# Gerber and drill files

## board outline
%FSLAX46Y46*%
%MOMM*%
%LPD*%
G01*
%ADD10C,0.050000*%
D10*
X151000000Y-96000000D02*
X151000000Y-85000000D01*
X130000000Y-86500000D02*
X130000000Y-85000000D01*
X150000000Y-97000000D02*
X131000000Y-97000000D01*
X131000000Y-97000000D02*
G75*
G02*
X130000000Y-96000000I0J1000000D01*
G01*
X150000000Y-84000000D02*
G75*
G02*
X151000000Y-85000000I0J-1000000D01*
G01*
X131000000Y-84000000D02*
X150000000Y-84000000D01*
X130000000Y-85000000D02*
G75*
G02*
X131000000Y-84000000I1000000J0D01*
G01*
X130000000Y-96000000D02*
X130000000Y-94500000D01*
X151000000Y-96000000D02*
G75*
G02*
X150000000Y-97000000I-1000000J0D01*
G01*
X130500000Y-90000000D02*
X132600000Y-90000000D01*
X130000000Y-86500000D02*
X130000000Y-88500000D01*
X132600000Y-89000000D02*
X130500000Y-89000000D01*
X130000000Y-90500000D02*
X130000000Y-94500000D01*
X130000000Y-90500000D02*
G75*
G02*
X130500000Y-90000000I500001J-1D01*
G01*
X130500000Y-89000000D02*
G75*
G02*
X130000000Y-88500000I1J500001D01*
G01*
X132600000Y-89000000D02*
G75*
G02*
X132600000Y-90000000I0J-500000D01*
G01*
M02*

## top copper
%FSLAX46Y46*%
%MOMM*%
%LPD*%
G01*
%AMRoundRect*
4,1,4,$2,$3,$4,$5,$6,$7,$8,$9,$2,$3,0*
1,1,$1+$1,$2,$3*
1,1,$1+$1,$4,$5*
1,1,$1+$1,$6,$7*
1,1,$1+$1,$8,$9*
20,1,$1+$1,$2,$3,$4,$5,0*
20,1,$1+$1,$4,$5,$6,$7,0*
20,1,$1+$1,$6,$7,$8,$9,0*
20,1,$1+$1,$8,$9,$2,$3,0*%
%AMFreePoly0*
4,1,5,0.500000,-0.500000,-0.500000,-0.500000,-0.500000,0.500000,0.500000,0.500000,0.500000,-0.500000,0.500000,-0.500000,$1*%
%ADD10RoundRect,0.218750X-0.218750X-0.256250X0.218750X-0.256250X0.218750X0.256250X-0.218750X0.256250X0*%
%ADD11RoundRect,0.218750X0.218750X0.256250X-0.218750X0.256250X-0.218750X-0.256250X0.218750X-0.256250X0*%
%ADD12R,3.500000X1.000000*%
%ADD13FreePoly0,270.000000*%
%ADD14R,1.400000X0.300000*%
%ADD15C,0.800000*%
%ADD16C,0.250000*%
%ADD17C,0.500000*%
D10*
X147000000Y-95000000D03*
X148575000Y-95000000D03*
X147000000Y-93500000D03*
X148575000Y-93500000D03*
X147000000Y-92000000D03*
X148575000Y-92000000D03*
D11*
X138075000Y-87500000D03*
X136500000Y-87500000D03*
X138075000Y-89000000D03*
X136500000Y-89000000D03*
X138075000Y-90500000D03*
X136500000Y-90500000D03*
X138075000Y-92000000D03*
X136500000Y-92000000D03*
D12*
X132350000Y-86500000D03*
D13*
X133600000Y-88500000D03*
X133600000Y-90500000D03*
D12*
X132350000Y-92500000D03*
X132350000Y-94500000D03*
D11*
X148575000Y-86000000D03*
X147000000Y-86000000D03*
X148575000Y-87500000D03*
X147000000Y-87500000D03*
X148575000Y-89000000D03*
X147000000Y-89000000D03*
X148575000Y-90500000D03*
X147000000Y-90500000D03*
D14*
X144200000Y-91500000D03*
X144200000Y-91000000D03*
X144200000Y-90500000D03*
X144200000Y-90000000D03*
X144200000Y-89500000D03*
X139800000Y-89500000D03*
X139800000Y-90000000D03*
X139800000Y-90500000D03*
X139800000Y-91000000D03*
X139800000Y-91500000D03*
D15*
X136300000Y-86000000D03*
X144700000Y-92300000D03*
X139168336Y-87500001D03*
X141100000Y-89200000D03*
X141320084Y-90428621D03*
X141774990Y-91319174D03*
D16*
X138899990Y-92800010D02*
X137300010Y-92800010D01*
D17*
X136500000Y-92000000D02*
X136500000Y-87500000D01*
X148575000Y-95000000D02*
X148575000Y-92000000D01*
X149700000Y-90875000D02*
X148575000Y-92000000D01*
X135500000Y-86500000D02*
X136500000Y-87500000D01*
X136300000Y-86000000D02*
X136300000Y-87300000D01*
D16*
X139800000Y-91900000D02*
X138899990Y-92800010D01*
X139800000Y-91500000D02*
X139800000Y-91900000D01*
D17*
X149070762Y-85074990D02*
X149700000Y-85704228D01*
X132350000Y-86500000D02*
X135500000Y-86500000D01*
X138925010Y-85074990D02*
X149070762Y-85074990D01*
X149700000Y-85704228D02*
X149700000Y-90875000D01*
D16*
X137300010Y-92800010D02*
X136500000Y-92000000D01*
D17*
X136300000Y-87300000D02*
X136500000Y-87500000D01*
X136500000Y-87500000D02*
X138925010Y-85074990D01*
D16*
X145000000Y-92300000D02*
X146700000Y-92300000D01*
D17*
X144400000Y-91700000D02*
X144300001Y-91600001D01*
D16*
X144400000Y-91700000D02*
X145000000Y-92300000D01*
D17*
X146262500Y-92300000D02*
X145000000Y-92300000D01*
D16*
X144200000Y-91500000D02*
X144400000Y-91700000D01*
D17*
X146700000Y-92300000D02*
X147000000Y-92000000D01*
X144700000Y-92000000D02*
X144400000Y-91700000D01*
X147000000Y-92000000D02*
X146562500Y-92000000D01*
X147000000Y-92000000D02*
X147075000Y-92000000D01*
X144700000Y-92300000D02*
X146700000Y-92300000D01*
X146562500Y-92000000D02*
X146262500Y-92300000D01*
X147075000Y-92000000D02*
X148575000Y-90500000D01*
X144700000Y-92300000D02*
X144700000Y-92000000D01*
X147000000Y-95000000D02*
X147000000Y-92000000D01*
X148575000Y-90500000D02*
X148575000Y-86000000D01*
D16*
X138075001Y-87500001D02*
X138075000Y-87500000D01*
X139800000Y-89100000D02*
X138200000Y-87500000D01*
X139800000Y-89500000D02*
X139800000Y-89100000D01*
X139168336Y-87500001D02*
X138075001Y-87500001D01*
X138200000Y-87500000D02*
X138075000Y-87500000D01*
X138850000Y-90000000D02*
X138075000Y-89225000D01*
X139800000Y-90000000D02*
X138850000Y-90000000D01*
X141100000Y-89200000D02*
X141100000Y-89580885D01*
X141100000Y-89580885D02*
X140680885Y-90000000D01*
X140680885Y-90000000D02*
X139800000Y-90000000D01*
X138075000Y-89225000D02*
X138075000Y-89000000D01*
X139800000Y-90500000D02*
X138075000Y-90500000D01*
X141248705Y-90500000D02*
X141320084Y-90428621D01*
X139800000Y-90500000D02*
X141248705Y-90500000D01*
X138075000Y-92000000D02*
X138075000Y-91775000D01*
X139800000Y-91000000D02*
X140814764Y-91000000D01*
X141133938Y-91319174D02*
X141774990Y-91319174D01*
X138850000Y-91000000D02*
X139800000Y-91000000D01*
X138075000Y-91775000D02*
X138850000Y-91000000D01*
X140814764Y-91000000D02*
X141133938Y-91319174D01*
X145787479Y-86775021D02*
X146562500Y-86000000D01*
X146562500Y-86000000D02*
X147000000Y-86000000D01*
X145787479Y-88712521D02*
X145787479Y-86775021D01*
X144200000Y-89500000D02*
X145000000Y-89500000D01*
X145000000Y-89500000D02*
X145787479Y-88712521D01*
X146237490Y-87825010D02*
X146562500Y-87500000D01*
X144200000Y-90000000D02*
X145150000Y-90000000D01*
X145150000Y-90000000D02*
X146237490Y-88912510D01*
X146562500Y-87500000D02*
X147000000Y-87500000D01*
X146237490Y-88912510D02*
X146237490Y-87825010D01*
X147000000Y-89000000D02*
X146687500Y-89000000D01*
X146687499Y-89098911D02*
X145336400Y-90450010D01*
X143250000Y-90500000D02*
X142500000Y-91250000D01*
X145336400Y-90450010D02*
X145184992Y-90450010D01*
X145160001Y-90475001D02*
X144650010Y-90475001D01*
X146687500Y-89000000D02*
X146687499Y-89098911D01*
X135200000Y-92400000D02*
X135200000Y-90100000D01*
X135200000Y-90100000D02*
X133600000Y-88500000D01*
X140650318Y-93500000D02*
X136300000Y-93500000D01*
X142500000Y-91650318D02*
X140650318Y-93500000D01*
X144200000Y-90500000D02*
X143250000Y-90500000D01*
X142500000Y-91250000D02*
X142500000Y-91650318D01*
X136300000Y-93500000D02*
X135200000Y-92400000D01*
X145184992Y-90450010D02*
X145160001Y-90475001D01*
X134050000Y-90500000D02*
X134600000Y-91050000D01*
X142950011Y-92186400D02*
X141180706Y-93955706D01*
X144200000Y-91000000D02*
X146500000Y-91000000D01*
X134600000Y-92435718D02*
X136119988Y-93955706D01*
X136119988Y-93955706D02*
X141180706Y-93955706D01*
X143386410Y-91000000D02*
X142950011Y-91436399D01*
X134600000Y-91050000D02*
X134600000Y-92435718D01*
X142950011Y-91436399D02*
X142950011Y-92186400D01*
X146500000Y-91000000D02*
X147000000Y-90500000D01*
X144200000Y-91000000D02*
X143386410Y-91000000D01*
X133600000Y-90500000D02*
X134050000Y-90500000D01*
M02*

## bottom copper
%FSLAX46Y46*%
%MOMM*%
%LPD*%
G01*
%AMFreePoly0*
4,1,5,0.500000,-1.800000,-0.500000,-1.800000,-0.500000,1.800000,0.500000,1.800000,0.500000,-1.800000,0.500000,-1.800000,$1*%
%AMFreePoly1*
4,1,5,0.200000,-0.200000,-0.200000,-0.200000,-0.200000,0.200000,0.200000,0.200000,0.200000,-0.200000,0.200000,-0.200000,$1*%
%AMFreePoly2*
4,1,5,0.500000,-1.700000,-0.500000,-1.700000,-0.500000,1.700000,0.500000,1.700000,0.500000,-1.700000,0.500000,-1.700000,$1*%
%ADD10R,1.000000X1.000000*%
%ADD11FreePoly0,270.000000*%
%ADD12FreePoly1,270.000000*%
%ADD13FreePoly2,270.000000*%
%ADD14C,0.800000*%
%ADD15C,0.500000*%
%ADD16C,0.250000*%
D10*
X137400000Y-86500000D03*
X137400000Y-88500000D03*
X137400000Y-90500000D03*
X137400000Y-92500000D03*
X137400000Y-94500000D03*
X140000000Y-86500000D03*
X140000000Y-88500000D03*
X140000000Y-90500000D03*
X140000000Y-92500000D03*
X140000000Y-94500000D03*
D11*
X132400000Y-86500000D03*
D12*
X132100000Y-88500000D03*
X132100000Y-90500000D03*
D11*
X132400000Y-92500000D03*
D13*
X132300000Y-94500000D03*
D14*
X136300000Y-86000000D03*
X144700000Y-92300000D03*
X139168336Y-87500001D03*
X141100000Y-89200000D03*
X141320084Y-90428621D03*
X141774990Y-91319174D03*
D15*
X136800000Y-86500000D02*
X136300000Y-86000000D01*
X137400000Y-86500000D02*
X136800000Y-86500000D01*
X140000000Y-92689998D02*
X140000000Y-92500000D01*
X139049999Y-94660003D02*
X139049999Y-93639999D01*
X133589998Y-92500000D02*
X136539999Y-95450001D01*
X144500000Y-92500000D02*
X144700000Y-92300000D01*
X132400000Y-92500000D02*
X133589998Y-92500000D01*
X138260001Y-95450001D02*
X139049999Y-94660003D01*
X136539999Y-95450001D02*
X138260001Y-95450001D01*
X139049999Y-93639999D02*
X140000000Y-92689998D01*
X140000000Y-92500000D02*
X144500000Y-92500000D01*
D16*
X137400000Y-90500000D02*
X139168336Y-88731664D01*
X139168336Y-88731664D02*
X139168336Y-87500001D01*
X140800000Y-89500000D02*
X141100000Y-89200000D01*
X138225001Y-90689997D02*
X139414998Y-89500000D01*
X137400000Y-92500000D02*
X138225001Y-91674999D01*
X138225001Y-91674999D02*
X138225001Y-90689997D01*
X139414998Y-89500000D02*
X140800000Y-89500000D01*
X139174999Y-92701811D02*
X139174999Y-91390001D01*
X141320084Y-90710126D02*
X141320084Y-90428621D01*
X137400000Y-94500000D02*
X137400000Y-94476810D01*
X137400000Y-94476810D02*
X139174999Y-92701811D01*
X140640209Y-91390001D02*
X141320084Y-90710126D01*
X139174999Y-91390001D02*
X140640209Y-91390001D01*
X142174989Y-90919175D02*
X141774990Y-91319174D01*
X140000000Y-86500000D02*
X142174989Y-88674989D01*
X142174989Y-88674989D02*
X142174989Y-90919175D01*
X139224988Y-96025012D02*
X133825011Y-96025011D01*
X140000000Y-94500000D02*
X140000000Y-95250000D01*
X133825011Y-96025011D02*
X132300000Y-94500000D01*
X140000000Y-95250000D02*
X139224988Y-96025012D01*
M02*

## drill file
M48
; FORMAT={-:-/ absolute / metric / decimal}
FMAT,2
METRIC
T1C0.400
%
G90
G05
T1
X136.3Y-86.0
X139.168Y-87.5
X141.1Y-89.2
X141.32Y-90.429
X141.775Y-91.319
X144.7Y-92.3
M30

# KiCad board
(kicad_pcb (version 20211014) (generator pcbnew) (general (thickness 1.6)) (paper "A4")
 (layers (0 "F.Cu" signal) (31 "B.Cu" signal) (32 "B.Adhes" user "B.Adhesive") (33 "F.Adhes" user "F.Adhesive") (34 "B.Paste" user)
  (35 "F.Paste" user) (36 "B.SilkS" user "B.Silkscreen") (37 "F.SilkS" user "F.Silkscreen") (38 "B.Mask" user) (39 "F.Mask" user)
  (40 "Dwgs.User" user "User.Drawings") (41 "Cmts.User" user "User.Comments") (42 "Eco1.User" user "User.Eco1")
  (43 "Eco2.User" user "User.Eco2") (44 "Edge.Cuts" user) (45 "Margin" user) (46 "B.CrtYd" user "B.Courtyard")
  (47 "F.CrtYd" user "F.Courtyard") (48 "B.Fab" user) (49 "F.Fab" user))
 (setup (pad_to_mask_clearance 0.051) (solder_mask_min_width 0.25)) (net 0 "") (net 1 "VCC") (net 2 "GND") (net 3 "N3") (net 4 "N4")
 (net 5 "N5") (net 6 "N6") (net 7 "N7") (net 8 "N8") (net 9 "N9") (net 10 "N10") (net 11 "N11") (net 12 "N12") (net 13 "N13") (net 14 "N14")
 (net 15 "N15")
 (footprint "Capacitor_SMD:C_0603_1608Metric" (layer "F.Cu") (at 147.7875 95)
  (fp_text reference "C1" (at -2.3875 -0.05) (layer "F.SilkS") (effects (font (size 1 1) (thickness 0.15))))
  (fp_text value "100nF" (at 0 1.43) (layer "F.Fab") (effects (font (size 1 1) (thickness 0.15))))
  (pad "1" smd roundrect locked (at -0.7875 0) (size 0.875 0.95) (layers "F.Cu" "F.Paste" "F.Mask") (roundrect_rratio 0.25) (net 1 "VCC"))
  (pad "2" smd roundrect locked (at 0.7875 0) (size 0.875 0.95) (layers "F.Cu" "F.Paste" "F.Mask") (roundrect_rratio 0.25) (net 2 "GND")))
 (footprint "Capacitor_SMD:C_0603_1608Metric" (layer "F.Cu") (at 147.7875 93.5)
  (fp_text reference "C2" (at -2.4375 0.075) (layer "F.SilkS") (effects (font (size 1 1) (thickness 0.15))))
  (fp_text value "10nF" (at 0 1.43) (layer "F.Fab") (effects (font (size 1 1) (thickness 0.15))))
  (pad "1" smd roundrect locked (at -0.7875 0) (size 0.875 0.95) (layers "F.Cu" "F.Paste" "F.Mask") (roundrect_rratio 0.25) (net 1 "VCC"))
  (pad "2" smd roundrect locked (at 0.7875 0) (size 0.875 0.95) (layers "F.Cu" "F.Paste" "F.Mask") (roundrect_rratio 0.25) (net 2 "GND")))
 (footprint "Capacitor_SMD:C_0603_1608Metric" (layer "F.Cu") (at 147.7875 92)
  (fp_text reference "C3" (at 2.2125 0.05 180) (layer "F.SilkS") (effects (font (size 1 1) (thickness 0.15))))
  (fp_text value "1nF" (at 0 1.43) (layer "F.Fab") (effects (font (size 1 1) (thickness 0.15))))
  (pad "1" smd roundrect locked (at -0.7875 0) (size 0.875 0.95) (layers "F.Cu" "F.Paste" "F.Mask") (roundrect_rratio 0.25) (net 1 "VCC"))
  (pad "2" smd roundrect locked (at 0.7875 0) (size 0.875 0.95) (layers "F.Cu" "F.Paste" "F.Mask") (roundrect_rratio 0.25) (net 2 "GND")))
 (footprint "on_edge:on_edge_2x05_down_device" (layer "F.Cu") (at 138.5 90.5 -90)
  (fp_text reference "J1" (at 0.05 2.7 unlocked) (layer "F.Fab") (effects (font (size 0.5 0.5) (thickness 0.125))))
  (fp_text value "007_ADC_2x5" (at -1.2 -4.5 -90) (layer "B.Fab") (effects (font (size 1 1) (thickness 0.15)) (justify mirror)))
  (pad "1" smd rect (at -4 1.1 90) (size 1 1) (layers "B.Cu" "B.Mask") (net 2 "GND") (zone_connect 0))
  (pad "2" smd rect (at -2 1.1 90) (size 1 1) (layers "B.Cu" "B.Mask") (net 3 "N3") (zone_connect 0))
  (pad "3" smd rect (at 0 1.1 90) (size 1 1) (layers "B.Cu" "B.Mask") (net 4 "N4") (zone_connect 0))
  (pad "4" smd rect (at 2 1.1 90) (size 1 1) (layers "B.Cu" "B.Mask") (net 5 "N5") (zone_connect 0))
  (pad "5" smd rect (at 4 1.1 90) (size 1 1) (layers "B.Cu" "B.Mask") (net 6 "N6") (zone_connect 0))
  (pad "6" smd rect (at -4 -1.5 270) (size 1 1) (layers "B.Cu" "B.Mask") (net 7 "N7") (zone_connect 0))
  (pad "7" smd rect (at -2 -1.5 270) (size 1 1) (layers "B.Cu" "B.Mask") (zone_connect 0))
  (pad "8" smd rect (at 0 -1.5 270) (size 1 1) (layers "B.Cu" "B.Mask") (zone_connect 0))
  (pad "9" smd rect (at 2 -1.5 270) (size 1 1) (layers "B.Cu" "B.Mask") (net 1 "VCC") (zone_connect 0))
  (pad "10" smd rect (at 4 -1.5 270) (size 1 1) (layers "B.Cu" "B.Mask") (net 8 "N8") (zone_connect 0)))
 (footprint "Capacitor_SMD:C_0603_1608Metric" (layer "F.Cu") (at 137.2875 87.5 180)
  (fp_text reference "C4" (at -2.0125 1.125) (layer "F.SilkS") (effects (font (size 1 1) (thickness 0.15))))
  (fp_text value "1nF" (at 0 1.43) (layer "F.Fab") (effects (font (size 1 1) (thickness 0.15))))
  (pad "1" smd roundrect locked (at -0.7875 0 180) (size 0.875 0.95) (layers "F.Cu" "F.Paste" "F.Mask") (roundrect_rratio 0.25) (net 4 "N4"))
  (pad "2" smd roundrect locked (at 0.7875 0 180) (size 0.875 0.95) (layers "F.Cu" "F.Paste" "F.Mask") (roundrect_rratio 0.25) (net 2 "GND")))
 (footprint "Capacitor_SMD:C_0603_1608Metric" (layer "F.Cu") (at 137.2875 89 180)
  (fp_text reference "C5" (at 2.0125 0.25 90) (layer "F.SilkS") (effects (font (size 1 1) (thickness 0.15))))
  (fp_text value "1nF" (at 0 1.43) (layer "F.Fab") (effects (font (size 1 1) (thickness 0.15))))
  (pad "1" smd roundrect locked (at -0.7875 0 180) (size 0.875 0.95) (layers "F.Cu" "F.Paste" "F.Mask") (roundrect_rratio 0.25) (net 5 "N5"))
  (pad "2" smd roundrect locked (at 0.7875 0 180) (size 0.875 0.95) (layers "F.Cu" "F.Paste" "F.Mask") (roundrect_rratio 0.25) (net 2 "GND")))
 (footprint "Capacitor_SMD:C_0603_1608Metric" (layer "F.Cu") (at 137.2875 90.5 180)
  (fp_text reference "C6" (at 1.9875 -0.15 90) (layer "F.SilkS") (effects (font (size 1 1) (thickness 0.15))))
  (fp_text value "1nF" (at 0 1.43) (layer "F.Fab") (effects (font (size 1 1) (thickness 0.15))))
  (pad "1" smd roundrect locked (at -0.7875 0 180) (size 0.875 0.95) (layers "F.Cu" "F.Paste" "F.Mask") (roundrect_rratio 0.25) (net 6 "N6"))
  (pad "2" smd roundrect locked (at 0.7875 0 180) (size 0.875 0.95) (layers "F.Cu" "F.Paste" "F.Mask") (roundrect_rratio 0.25) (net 2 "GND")))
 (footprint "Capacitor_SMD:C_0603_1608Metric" (layer "F.Cu") (at 137.2875 92 180)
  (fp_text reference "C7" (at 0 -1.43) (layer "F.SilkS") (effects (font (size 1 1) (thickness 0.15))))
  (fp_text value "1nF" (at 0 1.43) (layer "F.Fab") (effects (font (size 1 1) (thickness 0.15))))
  (pad "1" smd roundrect locked (at -0.7875 0 180) (size 0.875 0.95) (layers "F.Cu" "F.Paste" "F.Mask") (roundrect_rratio 0.25) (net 7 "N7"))
  (pad "2" smd roundrect locked (at 0.7875 0 180) (size 0.875 0.95) (layers "F.Cu" "F.Paste" "F.Mask") (roundrect_rratio 0.25) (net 2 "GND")))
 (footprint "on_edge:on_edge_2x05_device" (layer "F.Cu") (at 130 90.5 -90)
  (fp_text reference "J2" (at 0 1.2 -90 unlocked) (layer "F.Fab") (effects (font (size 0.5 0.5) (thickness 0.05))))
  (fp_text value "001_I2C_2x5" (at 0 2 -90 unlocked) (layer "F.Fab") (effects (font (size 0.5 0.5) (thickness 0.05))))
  (fp_line (start -0.5 -0.5) (end -0.5 -2.6) (layer "Edge.Cuts") (width 0.05))
  (fp_line (start -4 0) (end -2 0) (layer "Edge.Cuts") (width 0.05))
  (fp_line (start -1.5 -2.6) (end -1.5 -0.5) (layer "Edge.Cuts") (width 0.05))
  (fp_line (start 0 0) (end 4 0) (layer "Edge.Cuts") (width 0.05))
  (fp_arc (start 0 0) (mid -0.353553 -0.146447) (end -0.5 -0.5) (layer "Edge.Cuts") (width 0.05))
  (fp_arc (start -1.5 -0.5) (mid -1.646447 -0.146447) (end -2 0) (layer "Edge.Cuts") (width 0.05))
  (fp_arc (start -1.5 -2.6) (mid -1 -3.1) (end -0.5 -2.6) (layer "Edge.Cuts") (width 0.05))
  (pad "1" smd rect locked (at -4 -2.35 90) (size 1 3.5) (layers "F.Cu" "F.Mask") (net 2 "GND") (zone_connect 0))
  (pad "2" smd custom locked (at -2 -3.6 270) (size 1 1) (layers "F.Cu" "F.Mask") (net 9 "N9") (zone_connect 0)
   (options (clearance outline) (anchor rect)) (primitives))
  (pad "3" smd custom locked (at 0 -3.6 270) (size 1 1) (layers "F.Cu" "F.Mask") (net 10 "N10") (zone_connect 0)
   (options (clearance outline) (anchor rect)) (primitives))
  (pad "4" smd rect locked (at 2 -2.35 90) (size 1 3.5) (layers "F.Cu" "F.Mask") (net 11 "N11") (zone_connect 0))
  (pad "5" smd rect locked (at 4 -2.35 90) (size 1 3.5) (layers "F.Cu" "F.Mask") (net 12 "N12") (zone_connect 0))
  (pad "6" smd custom locked (at -4 -2.4 270) (size 1 3.6) (layers "B.Cu" "B.Mask") (zone_connect 0)
   (options (clearance outline) (anchor rect)) (primitives))
  (pad "7" smd custom locked (at -2 -2.1 270) (size 0.4 0.4) (layers "B.Cu" "B.Mask") (zone_connect 0)
   (options (clearance outline) (anchor rect)) (primitives))
  (pad "8" smd custom locked (at 0 -2.1 270) (size 0.4 0.4) (layers "B.Cu" "B.Mask") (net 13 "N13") (zone_connect 0)
   (options (clearance outline) (anchor rect)) (primitives))
  (pad "9" smd custom locked (at 2 -2.4 270) (size 1 3.6) (layers "B.Cu" "B.Mask") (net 1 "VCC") (zone_connect 0)
   (options (clearance outline) (anchor rect)) (primitives))
  (pad "10" smd custom locked (at 4 -2.3 270) (size 1 3.4) (layers "B.Cu" "B.Mask") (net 8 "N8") (zone_connect 0)
   (options (clearance outline) (anchor rect)) (primitives)))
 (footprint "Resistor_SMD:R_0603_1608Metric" (layer "F.Cu") (at 147.7875 86 180)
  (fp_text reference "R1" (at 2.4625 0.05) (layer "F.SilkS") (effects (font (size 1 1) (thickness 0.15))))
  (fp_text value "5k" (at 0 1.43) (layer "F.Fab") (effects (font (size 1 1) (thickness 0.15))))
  (pad "1" smd roundrect locked (at -0.7875 0 180) (size 0.875 0.95) (layers "F.Cu" "F.Paste" "F.Mask") (roundrect_rratio 0.25)
   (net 1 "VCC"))
  (pad "2" smd roundrect locked (at 0.7875 0 180) (size 0.875 0.95) (layers "F.Cu" "F.Paste" "F.Mask") (roundrect_rratio 0.25)
   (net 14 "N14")))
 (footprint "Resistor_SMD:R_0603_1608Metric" (layer "F.Cu") (at 147.7875 87.5 180)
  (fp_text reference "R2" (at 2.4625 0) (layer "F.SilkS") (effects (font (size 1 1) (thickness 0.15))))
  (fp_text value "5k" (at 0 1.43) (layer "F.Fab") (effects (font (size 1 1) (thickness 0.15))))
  (pad "1" smd roundrect locked (at -0.7875 0 180) (size 0.875 0.95) (layers "F.Cu" "F.Paste" "F.Mask") (roundrect_rratio 0.25)
   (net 1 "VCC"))
  (pad "2" smd roundrect locked (at 0.7875 0 180) (size 0.875 0.95) (layers "F.Cu" "F.Paste" "F.Mask") (roundrect_rratio 0.25)
   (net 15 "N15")))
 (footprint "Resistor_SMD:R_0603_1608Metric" (layer "F.Cu") (at 147.7875 89 180)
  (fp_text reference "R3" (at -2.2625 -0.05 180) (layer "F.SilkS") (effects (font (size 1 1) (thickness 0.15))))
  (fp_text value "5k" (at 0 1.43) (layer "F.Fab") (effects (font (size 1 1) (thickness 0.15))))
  (pad "1" smd roundrect locked (at -0.7875 0 180) (size 0.875 0.95) (layers "F.Cu" "F.Paste" "F.Mask") (roundrect_rratio 0.25)
   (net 1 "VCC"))
  (pad "2" smd roundrect locked (at 0.7875 0 180) (size 0.875 0.95) (layers "F.Cu" "F.Paste" "F.Mask") (roundrect_rratio 0.25) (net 9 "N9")))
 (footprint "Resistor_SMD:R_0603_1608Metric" (layer "F.Cu") (at 147.7875 90.5 180)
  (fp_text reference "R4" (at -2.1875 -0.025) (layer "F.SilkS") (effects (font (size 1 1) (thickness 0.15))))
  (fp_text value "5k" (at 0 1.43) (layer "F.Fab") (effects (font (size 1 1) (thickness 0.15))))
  (pad "1" smd roundrect locked (at -0.7875 0 180) (size 0.875 0.95) (layers "F.Cu" "F.Paste" "F.Mask") (roundrect_rratio 0.25)
   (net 1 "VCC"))
  (pad "2" smd roundrect locked (at 0.7875 0 180) (size 0.875 0.95) (layers "F.Cu" "F.Paste" "F.Mask") (roundrect_rratio 0.25)
   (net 10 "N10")))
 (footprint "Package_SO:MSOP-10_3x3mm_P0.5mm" (layer "F.Cu") (at 142 90.5 180)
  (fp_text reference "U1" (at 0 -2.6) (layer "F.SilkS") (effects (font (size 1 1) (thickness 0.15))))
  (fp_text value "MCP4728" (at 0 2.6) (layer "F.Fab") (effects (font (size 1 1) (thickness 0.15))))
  (pad "1" smd rect locked (at -2.2 -1 180) (size 1.4 0.3) (layers "F.Cu" "F.Paste" "F.Mask") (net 1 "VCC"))
  (pad "2" smd rect locked (at -2.2 -0.5 180) (size 1.4 0.3) (layers "F.Cu" "F.Paste" "F.Mask") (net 10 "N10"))
  (pad "3" smd rect locked (at -2.2 0 180) (size 1.4 0.3) (layers "F.Cu" "F.Paste" "F.Mask") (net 9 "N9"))
  (pad "4" smd rect locked (at -2.2 0.5 180) (size 1.4 0.3) (layers "F.Cu" "F.Paste" "F.Mask") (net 15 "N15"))
  (pad "5" smd rect locked (at -2.2 1 180) (size 1.4 0.3) (layers "F.Cu" "F.Paste" "F.Mask") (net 14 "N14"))
  (pad "6" smd rect locked (at 2.2 1 180) (size 1.4 0.3) (layers "F.Cu" "F.Paste" "F.Mask") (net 4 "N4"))
  (pad "7" smd rect locked (at 2.2 0.5 180) (size 1.4 0.3) (layers "F.Cu" "F.Paste" "F.Mask") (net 5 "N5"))
  (pad "8" smd rect locked (at 2.2 0 180) (size 1.4 0.3) (layers "F.Cu" "F.Paste" "F.Mask") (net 6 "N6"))
  (pad "9" smd rect locked (at 2.2 -0.5 180) (size 1.4 0.3) (layers "F.Cu" "F.Paste" "F.Mask") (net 7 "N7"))
  (pad "10" smd rect locked (at 2.2 -1 180) (size 1.4 0.3) (layers "F.Cu" "F.Paste" "F.Mask") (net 2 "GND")))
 (gr_line (start 151 96) (end 151 85) (layer "Edge.Cuts") (width 0.05))
 (gr_line (start 130 86.5) (end 130 85) (layer "Edge.Cuts") (width 0.05))
 (gr_line (start 150 97) (end 131 97) (layer "Edge.Cuts") (width 0.05))
 (gr_arc (start 131 97) (mid 130.292893 96.707107) (end 130 96) (layer "Edge.Cuts") (width 0.05))
 (gr_arc (start 150 84) (mid 150.707107 84.292893) (end 151 85) (layer "Edge.Cuts") (width 0.05))
 (gr_line (start 131 84) (end 150 84) (layer "Edge.Cuts") (width 0.05))
 (gr_arc (start 130 85) (mid 130.292893 84.292893) (end 131 84) (layer "Edge.Cuts") (width 0.05))
 (gr_line (start 130 96) (end 130 94.5) (layer "Edge.Cuts") (width 0.05))
 (gr_arc (start 151 96) (mid 150.707107 96.707107) (end 150 97) (layer "Edge.Cuts") (width 0.05))
 (segment (start 138.89999 92.80001) (end 137.30001 92.80001) (width 0.25) (layer "F.Cu") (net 2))
 (segment (start 136.5 92) (end 136.5 87.5) (width 0.5) (layer "F.Cu") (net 2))
 (segment (start 148.575 95) (end 148.575 92) (width 0.5) (layer "F.Cu") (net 2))
 (segment (start 149.7 90.875) (end 148.575 92) (width 0.5) (layer "F.Cu") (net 2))
 (segment (start 135.5 86.5) (end 136.5 87.5) (width 0.5) (layer "F.Cu") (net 2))
 (segment (start 136.3 86) (end 136.3 87.3) (width 0.5) (layer "F.Cu") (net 2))
 (segment (start 139.8 91.9) (end 138.89999 92.80001) (width 0.25) (layer "F.Cu") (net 2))
 (segment (start 139.8 91.5) (end 139.8 91.9) (width 0.25) (layer "F.Cu") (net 2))
 (segment (start 149.070762 85.07499) (end 149.7 85.704228) (width 0.5) (layer "F.Cu") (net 2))
 (segment (start 132.35 86.5) (end 135.5 86.5) (width 0.5) (layer "F.Cu") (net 2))
 (segment (start 138.92501 85.07499) (end 149.070762 85.07499) (width 0.5) (layer "F.Cu") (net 2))
 (segment (start 149.7 85.704228) (end 149.7 90.875) (width 0.5) (layer "F.Cu") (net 2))
 (segment (start 137.30001 92.80001) (end 136.5 92) (width 0.25) (layer "F.Cu") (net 2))
 (segment (start 136.3 87.3) (end 136.5 87.5) (width 0.5) (layer "F.Cu") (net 2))
 (segment (start 136.5 87.5) (end 138.92501 85.07499) (width 0.5) (layer "F.Cu") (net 2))
 (via (at 136.3 86) (size 0.8) (drill 0.4) (layers "F.Cu" "B.Cu") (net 2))
 (segment (start 136.8 86.5) (end 136.3 86) (width 0.5) (layer "B.Cu") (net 2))
 (segment (start 137.4 86.5) (end 136.8 86.5) (width 0.5) (layer "B.Cu") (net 2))
 (segment (start 145 92.3) (end 146.7 92.3) (width 0.25) (layer "F.Cu") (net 1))
 (segment (start 144.4 91.7) (end 144.300001 91.600001) (width 0.5) (layer "F.Cu") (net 1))
 (segment (start 144.4 91.7) (end 145 92.3) (width 0.25) (layer "F.Cu") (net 1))
 (segment (start 146.2625 92.3) (end 145 92.3) (width 0.5) (layer "F.Cu") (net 1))
 (segment (start 144.2 91.5) (end 144.4 91.7) (width 0.25) (layer "F.Cu") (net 1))
 (segment (start 146.7 92.3) (end 147 92) (width 0.5) (layer "F.Cu") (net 1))
 (segment (start 144.7 92) (end 144.4 91.7) (width 0.5) (layer "F.Cu") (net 1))
 (segment (start 147 92) (end 146.5625 92) (width 0.5) (layer "F.Cu") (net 1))
 (segment (start 147 92) (end 147.075 92) (width 0.5) (layer "F.Cu") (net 1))
 (segment (start 144.7 92.3) (end 146.7 92.3) (width 0.5) (layer "F.Cu") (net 1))
 (segment (start 146.5625 92) (end 146.2625 92.3) (width 0.5) (layer "F.Cu") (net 1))
 (segment (start 147.075 92) (end 148.575 90.5) (width 0.5) (layer "F.Cu") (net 1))
 (segment (start 144.7 92.3) (end 144.7 92) (width 0.5) (layer "F.Cu") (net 1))
 (segment (start 147 95) (end 147 92) (width 0.5) (layer "F.Cu") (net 1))
 (segment (start 148.575 90.5) (end 148.575 86) (width 0.5) (layer "F.Cu") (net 1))
 (via (at 144.7 92.3) (size 0.8) (drill 0.4) (layers "F.Cu" "B.Cu") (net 1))
 (segment (start 140 92.689998) (end 140 92.5) (width 0.5) (layer "B.Cu") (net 1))
 (segment (start 139.049999 94.660003) (end 139.049999 93.639999) (width 0.5) (layer "B.Cu") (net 1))
 (segment (start 133.589998 92.5) (end 136.539999 95.450001) (width 0.5) (layer "B.Cu") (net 1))
 (segment (start 144.5 92.5) (end 144.7 92.3) (width 0.5) (layer "B.Cu") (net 1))
 (segment (start 132.4 92.5) (end 133.589998 92.5) (width 0.5) (layer "B.Cu") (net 1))
 (segment (start 138.260001 95.450001) (end 139.049999 94.660003) (width 0.5) (layer "B.Cu") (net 1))
 (segment (start 136.539999 95.450001) (end 138.260001 95.450001) (width 0.5) (layer "B.Cu") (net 1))
 (segment (start 139.049999 93.639999) (end 140 92.689998) (width 0.5) (layer "B.Cu") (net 1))
 (segment (start 140 92.5) (end 144.5 92.5) (width 0.5) (layer "B.Cu") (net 1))
 (segment (start 138.075001 87.500001) (end 138.075 87.5) (width 0.25) (layer "F.Cu") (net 4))
 (segment (start 139.8 89.1) (end 138.2 87.5) (width 0.25) (layer "F.Cu") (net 4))
 (segment (start 139.8 89.5) (end 139.8 89.1) (width 0.25) (layer "F.Cu") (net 4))
 (segment (start 139.168336 87.500001) (end 138.075001 87.500001) (width 0.25) (layer "F.Cu") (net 4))
 (segment (start 138.2 87.5) (end 138.075 87.5) (width 0.25) (layer "F.Cu") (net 4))
 (via (at 139.168336 87.500001) (size 0.8) (drill 0.4) (layers "F.Cu" "B.Cu") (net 4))
 (segment (start 137.4 90.5) (end 139.168336 88.731664) (width 0.25) (layer "B.Cu") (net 4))
 (segment (start 139.168336 88.731664) (end 139.168336 87.500001) (width 0.25) (layer "B.Cu") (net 4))
 (segment (start 138.85 90) (end 138.075 89.225) (width 0.25) (layer "F.Cu") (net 5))
 (segment (start 139.8 90) (end 138.85 90) (width 0.25) (layer "F.Cu") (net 5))
 (segment (start 141.1 89.2) (end 141.1 89.580885) (width 0.25) (layer "F.Cu") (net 5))
 (segment (start 141.1 89.580885) (end 140.680885 90) (width 0.25) (layer "F.Cu") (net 5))
 (segment (start 140.680885 90) (end 139.8 90) (width 0.25) (layer "F.Cu") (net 5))
 (segment (start 138.075 89.225) (end 138.075 89) (width 0.25) (layer "F.Cu") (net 5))
 (via (at 141.1 89.2) (size 0.8) (drill 0.4) (layers "F.Cu" "B.Cu") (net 5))
 (segment (start 140.8 89.5) (end 141.1 89.2) (width 0.25) (layer "B.Cu") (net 5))
 (segment (start 138.225001 90.689997) (end 139.414998 89.5) (width 0.25) (layer "B.Cu") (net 5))
 (segment (start 137.4 92.5) (end 138.225001 91.674999) (width 0.25) (layer "B.Cu") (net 5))
 (segment (start 138.225001 91.674999) (end 138.225001 90.689997) (width 0.25) (layer "B.Cu") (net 5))
 (segment (start 139.414998 89.5) (end 140.8 89.5) (width 0.25) (layer "B.Cu") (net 5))
 (segment (start 139.8 90.5) (end 138.075 90.5) (width 0.25) (layer "F.Cu") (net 6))
 (segment (start 141.248705 90.5) (end 141.320084 90.428621) (width 0.25) (layer "F.Cu") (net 6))
 (segment (start 139.8 90.5) (end 141.248705 90.5) (width 0.25) (layer "F.Cu") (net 6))
 (via (at 141.320084 90.428621) (size 0.8) (drill 0.4) (layers "F.Cu" "B.Cu") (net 6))
 (segment (start 139.174999 92.701811) (end 139.174999 91.390001) (width 0.25) (layer "B.Cu") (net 6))
 (segment (start 141.320084 90.710126) (end 141.320084 90.428621) (width 0.25) (layer "B.Cu") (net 6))
 (segment (start 137.4 94.5) (end 137.4 94.47681) (width 0.25) (layer "B.Cu") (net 6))
 (segment (start 137.4 94.47681) (end 139.174999 92.701811) (width 0.25) (layer "B.Cu") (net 6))
 (segment (start 140.640209 91.390001) (end 141.320084 90.710126) (width 0.25) (layer "B.Cu") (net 6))
 (segment (start 139.174999 91.390001) (end 140.640209 91.390001) (width 0.25) (layer "B.Cu") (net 6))
 (segment (start 138.075 92) (end 138.075 91.775) (width 0.25) (layer "F.Cu") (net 7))
 (segment (start 139.8 91) (end 140.814764 91) (width 0.25) (layer "F.Cu") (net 7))
 (segment (start 141.133938 91.319174) (end 141.77499 91.319174) (width 0.25) (layer "F.Cu") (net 7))
 (segment (start 138.85 91) (end 139.8 91) (width 0.25) (layer "F.Cu") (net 7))
 (segment (start 138.075 91.775) (end 138.85 91) (width 0.25) (layer "F.Cu") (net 7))
 (segment (start 140.814764 91) (end 141.133938 91.319174) (width 0.25) (layer "F.Cu") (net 7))
 (via (at 141.77499 91.319174) (size 0.8) (drill 0.4) (layers "F.Cu" "B.Cu") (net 7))
 (segment (start 142.174989 90.919175) (end 141.77499 91.319174) (width 0.25) (layer "B.Cu") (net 7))
 (segment (start 140 86.5) (end 142.174989 88.674989) (width 0.25) (layer "B.Cu") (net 7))
 (segment (start 142.174989 88.674989) (end 142.174989 90.919175) (width 0.25) (layer "B.Cu") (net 7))
 (segment (start 139.224988 96.025012) (end 133.825011 96.025011) (width 0.25) (layer "B.Cu") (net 8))
 (segment (start 140 94.5) (end 140 95.25) (width 0.25) (layer "B.Cu") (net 8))
 (segment (start 133.825011 96.025011) (end 132.3 94.5) (width 0.25) (layer "B.Cu") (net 8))
 (segment (start 140 95.25) (end 139.224988 96.025012) (width 0.25) (layer "B.Cu") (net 8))
 (segment (start 145.787479 86.775021) (end 146.5625 86) (width 0.25) (layer "F.Cu") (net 14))
 (segment (start 146.5625 86) (end 147 86) (width 0.25) (layer "F.Cu") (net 14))
 (segment (start 145.787479 88.712521) (end 145.787479 86.775021) (width 0.25) (layer "F.Cu") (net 14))
 (segment (start 144.2 89.5) (end 145 89.5) (width 0.25) (layer "F.Cu") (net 14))
 (segment (start 145 89.5) (end 145.787479 88.712521) (width 0.25) (layer "F.Cu") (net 14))
 (segment (start 146.23749 87.82501) (end 146.5625 87.5) (width 0.25) (layer "F.Cu") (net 15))
 (segment (start 144.2 90) (end 145.15 90) (width 0.25) (layer "F.Cu") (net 15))
 (segment (start 145.15 90) (end 146.23749 88.91251) (width 0.25) (layer "F.Cu") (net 15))
 (segment (start 146.5625 87.5) (end 147 87.5) (width 0.25) (layer "F.Cu") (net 15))
 (segment (start 146.23749 88.91251) (end 146.23749 87.82501) (width 0.25) (layer "F.Cu") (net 15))
 (segment (start 147 89) (end 146.6875 89) (width 0.25) (layer "F.Cu") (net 9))
 (segment (start 146.687499 89.098911) (end 145.3364 90.45001) (width 0.25) (layer "F.Cu") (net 9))
 (segment (start 143.25 90.5) (end 142.5 91.25) (width 0.25) (layer "F.Cu") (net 9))
 (segment (start 145.3364 90.45001) (end 145.184992 90.45001) (width 0.25) (layer "F.Cu") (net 9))
 (segment (start 145.160001 90.475001) (end 144.65001 90.475001) (width 0.25) (layer "F.Cu") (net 9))
 (segment (start 146.6875 89) (end 146.687499 89.098911) (width 0.25) (layer "F.Cu") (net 9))
 (segment (start 135.2 92.4) (end 135.2 90.1) (width 0.25) (layer "F.Cu") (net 9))
 (segment (start 135.2 90.1) (end 133.6 88.5) (width 0.25) (layer "F.Cu") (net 9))
 (segment (start 140.650318 93.5) (end 136.3 93.5) (width 0.25) (layer "F.Cu") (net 9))
 (segment (start 142.5 91.650318) (end 140.650318 93.5) (width 0.25) (layer "F.Cu") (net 9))
 (segment (start 144.2 90.5) (end 143.25 90.5) (width 0.25) (layer "F.Cu") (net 9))
 (segment (start 142.5 91.25) (end 142.5 91.650318) (width 0.25) (layer "F.Cu") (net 9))
 (segment (start 136.3 93.5) (end 135.2 92.4) (width 0.25) (layer "F.Cu") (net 9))
 (segment (start 145.184992 90.45001) (end 145.160001 90.475001) (width 0.25) (layer "F.Cu") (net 9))
 (segment (start 134.05 90.5) (end 134.6 91.05) (width 0.25) (layer "F.Cu") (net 10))
 (segment (start 142.950011 92.1864) (end 141.180706 93.955706) (width 0.25) (layer "F.Cu") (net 10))
 (segment (start 144.2 91) (end 146.5 91) (width 0.25) (layer "F.Cu") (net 10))
 (segment (start 134.6 92.435718) (end 136.119988 93.955706) (width 0.25) (layer "F.Cu") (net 10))
 (segment (start 136.119988 93.955706) (end 141.180706 93.955706) (width 0.25) (layer "F.Cu") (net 10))
 (segment (start 143.38641 91) (end 142.950011 91.436399) (width 0.25) (layer "F.Cu") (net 10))
 (segment (start 134.6 91.05) (end 134.6 92.435718) (width 0.25) (layer "F.Cu") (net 10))
 (segment (start 142.950011 91.436399) (end 142.950011 92.1864) (width 0.25) (layer "F.Cu") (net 10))
 (segment (start 146.5 91) (end 147 90.5) (width 0.25) (layer "F.Cu") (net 10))
 (segment (start 144.2 91) (end 143.38641 91) (width 0.25) (layer "F.Cu") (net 10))
 (segment (start 133.6 90.5) (end 134.05 90.5) (width 0.25) (layer "F.Cu") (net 10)))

